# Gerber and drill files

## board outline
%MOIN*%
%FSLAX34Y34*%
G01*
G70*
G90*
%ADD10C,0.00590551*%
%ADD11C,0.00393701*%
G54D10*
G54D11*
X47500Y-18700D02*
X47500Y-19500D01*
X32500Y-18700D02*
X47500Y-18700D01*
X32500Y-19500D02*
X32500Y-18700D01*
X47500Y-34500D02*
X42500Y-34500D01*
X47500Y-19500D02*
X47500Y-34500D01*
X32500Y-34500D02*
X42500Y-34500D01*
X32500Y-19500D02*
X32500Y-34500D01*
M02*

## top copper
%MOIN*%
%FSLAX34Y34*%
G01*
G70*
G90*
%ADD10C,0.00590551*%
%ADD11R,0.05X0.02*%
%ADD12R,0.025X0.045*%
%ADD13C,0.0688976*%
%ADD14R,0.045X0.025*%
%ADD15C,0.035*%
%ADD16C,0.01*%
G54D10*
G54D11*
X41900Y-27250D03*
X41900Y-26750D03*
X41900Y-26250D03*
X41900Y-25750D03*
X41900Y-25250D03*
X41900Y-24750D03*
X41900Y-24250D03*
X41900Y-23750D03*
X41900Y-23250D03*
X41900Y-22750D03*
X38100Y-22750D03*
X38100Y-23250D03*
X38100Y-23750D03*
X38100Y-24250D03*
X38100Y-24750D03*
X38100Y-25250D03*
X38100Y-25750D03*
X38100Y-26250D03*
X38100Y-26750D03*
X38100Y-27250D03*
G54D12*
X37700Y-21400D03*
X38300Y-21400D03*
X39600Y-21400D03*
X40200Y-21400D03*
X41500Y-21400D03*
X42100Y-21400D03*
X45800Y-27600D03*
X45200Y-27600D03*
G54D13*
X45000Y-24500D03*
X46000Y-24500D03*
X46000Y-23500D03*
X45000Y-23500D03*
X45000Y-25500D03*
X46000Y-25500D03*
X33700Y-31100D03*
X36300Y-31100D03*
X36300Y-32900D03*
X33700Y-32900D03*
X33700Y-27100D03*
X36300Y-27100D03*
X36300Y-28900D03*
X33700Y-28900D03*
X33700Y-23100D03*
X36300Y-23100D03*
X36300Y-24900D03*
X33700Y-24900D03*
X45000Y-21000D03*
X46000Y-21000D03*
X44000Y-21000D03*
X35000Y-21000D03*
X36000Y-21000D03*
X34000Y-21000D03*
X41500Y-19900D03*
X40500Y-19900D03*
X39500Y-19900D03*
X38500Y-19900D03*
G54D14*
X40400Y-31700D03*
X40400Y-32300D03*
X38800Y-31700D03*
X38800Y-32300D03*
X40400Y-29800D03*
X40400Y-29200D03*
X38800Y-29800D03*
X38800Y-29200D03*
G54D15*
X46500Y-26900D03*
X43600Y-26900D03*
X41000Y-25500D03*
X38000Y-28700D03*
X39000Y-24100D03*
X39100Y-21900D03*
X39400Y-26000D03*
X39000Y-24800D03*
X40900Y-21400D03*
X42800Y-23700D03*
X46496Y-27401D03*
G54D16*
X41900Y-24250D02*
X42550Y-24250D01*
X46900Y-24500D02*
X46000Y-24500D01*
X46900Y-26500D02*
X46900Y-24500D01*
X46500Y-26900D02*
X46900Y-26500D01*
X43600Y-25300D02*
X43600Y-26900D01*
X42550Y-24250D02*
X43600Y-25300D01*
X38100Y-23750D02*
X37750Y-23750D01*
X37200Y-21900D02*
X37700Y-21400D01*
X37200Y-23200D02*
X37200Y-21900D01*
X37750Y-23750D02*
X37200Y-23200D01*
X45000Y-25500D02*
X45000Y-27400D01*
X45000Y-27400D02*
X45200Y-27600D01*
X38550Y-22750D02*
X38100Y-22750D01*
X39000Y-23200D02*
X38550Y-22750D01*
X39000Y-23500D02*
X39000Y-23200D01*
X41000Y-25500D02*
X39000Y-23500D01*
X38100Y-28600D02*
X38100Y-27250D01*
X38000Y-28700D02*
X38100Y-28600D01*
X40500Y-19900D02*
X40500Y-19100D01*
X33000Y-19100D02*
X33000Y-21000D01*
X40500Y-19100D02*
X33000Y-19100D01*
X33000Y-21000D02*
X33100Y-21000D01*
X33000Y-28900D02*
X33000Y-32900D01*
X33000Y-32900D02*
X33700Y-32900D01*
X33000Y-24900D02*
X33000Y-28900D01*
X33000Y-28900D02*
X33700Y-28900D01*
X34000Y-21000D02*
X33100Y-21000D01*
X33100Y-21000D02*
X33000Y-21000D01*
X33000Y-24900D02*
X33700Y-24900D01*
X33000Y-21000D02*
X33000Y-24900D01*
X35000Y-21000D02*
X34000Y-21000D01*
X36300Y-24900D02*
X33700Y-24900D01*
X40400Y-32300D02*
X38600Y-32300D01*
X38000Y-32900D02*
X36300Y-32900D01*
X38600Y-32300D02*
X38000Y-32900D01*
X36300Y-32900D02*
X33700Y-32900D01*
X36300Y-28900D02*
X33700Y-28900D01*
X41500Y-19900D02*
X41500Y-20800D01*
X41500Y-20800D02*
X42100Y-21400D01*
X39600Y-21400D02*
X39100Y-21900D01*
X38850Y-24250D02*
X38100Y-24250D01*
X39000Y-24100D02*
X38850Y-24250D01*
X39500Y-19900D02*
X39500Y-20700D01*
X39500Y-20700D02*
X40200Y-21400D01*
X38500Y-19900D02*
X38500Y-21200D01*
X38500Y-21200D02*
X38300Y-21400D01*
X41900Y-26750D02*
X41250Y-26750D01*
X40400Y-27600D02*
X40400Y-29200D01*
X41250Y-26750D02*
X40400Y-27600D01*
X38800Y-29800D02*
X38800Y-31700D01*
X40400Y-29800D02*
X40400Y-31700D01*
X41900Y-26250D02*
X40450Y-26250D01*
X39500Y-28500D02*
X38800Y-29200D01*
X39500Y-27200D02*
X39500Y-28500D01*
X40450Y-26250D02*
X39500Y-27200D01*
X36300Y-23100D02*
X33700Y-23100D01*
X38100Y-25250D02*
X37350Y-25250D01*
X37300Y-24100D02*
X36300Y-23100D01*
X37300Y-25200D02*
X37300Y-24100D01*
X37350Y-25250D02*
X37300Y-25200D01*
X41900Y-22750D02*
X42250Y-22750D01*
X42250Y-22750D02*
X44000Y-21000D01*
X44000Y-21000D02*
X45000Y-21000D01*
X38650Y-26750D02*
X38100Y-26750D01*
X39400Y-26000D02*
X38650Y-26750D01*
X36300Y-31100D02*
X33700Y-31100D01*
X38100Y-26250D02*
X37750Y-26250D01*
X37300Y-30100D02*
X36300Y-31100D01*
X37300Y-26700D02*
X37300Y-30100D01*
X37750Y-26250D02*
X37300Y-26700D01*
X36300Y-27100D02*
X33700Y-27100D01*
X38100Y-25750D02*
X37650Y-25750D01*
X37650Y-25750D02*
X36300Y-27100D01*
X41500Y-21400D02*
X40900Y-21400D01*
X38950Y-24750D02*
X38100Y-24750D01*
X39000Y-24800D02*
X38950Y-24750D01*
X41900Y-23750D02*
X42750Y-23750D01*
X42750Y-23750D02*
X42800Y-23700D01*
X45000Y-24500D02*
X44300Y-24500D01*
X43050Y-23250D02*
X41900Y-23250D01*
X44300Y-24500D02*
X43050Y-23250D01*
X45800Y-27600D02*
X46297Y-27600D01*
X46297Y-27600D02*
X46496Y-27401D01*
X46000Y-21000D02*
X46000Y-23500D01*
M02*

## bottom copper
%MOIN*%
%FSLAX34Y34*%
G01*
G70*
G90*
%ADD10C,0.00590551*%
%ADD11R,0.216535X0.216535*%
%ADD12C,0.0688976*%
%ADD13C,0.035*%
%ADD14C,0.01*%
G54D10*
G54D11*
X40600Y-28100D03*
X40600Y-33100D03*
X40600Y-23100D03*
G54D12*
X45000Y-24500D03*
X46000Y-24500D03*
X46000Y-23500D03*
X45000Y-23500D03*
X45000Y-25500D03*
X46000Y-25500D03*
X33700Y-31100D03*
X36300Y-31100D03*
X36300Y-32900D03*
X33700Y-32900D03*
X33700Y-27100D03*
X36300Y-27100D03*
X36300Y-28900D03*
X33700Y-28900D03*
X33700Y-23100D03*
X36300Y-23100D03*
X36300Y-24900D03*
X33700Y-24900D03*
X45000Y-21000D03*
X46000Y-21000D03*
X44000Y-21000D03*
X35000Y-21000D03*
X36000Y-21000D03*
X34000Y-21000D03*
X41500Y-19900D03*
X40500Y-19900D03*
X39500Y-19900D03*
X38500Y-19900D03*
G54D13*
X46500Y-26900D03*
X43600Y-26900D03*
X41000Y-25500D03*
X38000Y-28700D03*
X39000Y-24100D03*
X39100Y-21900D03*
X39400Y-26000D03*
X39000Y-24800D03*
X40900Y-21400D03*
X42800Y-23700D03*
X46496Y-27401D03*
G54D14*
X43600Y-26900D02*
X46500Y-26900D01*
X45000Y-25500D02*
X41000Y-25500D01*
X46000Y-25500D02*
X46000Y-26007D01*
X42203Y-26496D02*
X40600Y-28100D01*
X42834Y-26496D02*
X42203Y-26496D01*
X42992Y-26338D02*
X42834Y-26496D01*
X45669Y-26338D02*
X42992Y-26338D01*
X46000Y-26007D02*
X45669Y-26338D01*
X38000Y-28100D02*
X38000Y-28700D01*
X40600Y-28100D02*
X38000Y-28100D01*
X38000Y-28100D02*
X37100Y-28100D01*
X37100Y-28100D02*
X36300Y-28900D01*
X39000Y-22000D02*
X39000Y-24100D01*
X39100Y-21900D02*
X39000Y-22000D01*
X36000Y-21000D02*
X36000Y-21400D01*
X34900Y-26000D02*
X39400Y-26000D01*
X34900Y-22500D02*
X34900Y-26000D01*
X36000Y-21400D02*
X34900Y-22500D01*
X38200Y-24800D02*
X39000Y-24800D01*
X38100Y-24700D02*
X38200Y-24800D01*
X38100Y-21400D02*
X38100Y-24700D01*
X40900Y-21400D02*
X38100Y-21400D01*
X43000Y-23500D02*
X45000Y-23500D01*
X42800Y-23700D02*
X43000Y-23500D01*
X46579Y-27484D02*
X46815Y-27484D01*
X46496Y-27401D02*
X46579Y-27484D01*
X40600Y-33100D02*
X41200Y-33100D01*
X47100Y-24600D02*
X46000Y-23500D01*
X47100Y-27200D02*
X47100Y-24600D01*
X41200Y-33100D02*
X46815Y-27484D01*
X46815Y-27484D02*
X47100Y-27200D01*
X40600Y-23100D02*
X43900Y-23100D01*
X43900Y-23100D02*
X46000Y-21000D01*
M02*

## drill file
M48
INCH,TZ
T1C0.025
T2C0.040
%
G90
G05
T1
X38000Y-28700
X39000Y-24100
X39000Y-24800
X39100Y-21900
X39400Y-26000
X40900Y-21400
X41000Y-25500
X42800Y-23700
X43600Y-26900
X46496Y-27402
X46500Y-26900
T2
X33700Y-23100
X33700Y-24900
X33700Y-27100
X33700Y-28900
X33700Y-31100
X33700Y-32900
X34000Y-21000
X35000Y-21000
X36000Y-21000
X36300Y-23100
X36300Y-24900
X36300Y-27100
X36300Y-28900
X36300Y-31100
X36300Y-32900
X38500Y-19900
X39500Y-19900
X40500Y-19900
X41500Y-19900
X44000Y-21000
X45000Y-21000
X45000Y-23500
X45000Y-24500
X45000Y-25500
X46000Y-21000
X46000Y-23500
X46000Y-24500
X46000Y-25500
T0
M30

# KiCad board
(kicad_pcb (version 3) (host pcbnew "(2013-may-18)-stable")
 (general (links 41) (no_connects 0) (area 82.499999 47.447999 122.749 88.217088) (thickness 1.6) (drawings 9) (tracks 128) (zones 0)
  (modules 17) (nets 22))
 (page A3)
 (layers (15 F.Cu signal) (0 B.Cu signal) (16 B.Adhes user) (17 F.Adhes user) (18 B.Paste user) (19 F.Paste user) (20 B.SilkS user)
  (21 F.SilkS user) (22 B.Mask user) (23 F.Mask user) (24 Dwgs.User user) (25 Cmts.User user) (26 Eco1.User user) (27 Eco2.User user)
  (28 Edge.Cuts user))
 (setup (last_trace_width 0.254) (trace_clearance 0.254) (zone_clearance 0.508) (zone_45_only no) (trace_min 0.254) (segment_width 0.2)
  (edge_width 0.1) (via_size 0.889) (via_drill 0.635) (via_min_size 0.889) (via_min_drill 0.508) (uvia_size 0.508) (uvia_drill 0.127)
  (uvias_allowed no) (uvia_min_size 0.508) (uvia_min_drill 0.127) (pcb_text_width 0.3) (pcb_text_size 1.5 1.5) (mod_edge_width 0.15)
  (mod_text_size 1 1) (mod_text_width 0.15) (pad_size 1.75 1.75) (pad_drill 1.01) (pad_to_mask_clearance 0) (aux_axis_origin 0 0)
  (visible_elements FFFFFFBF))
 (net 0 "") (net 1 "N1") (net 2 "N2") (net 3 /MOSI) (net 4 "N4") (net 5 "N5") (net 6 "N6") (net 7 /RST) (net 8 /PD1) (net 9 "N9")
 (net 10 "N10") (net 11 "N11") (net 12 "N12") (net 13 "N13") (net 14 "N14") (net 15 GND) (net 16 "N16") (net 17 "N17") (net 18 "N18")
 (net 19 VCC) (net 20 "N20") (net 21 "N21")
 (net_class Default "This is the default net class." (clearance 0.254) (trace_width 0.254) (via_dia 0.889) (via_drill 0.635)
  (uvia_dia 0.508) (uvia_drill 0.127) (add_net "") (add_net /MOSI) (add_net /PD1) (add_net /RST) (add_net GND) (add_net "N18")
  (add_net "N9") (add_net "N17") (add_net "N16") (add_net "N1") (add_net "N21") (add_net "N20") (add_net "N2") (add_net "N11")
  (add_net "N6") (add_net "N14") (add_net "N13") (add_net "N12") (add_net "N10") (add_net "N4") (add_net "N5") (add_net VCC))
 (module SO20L (layer F.Cu) (at 101.6 63.5 270)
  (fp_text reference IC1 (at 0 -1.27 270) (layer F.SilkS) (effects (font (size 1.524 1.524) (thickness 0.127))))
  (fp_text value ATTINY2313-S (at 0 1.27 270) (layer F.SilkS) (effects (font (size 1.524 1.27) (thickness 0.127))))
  (pad 11 smd rect (at 5.715 -4.826 270) (size 0.508 1.27) (layers F.Cu F.Paste F.Mask))
  (pad 12 smd rect (at 4.445 -4.826 270) (size 0.508 1.27) (layers F.Cu F.Paste F.Mask) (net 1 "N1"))
  (pad 13 smd rect (at 3.175 -4.826 270) (size 0.508 1.27) (layers F.Cu F.Paste F.Mask) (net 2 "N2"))
  (pad 14 smd rect (at 1.905 -4.826 270) (size 0.508 1.27) (layers F.Cu F.Paste F.Mask))
  (pad 15 smd rect (at 0.635 -4.826 270) (size 0.508 1.27) (layers F.Cu F.Paste F.Mask))
  (pad 16 smd rect (at -0.635 -4.826 270) (size 0.508 1.27) (layers F.Cu F.Paste F.Mask))
  (pad 17 smd rect (at -1.905 -4.826 270) (size 0.508 1.27) (layers F.Cu F.Paste F.Mask) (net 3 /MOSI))
  (pad 18 smd rect (at -3.175 -4.826 270) (size 0.508 1.27) (layers F.Cu F.Paste F.Mask) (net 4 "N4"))
  (pad 19 smd rect (at -4.445 -4.826 270) (size 0.508 1.27) (layers F.Cu F.Paste F.Mask) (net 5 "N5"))
  (pad 20 smd rect (at -5.715 -4.826 270) (size 0.508 1.27) (layers F.Cu F.Paste F.Mask) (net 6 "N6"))
  (pad 1 smd rect (at -5.715 4.826 270) (size 0.508 1.27) (layers F.Cu F.Paste F.Mask) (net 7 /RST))
  (pad 2 smd rect (at -4.445 4.826 270) (size 0.508 1.27) (layers F.Cu F.Paste F.Mask))
  (pad 3 smd rect (at -3.175 4.826 270) (size 0.508 1.27) (layers F.Cu F.Paste F.Mask) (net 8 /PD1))
  (pad 4 smd rect (at -1.905 4.826 270) (size 0.508 1.27) (layers F.Cu F.Paste F.Mask) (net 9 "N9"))
  (pad 5 smd rect (at -0.635 4.826 270) (size 0.508 1.27) (layers F.Cu F.Paste F.Mask) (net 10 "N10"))
  (pad 6 smd rect (at 0.635 4.826 270) (size 0.508 1.27) (layers F.Cu F.Paste F.Mask) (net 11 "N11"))
  (pad 7 smd rect (at 1.905 4.826 270) (size 0.508 1.27) (layers F.Cu F.Paste F.Mask) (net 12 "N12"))
  (pad 8 smd rect (at 3.175 4.826 270) (size 0.508 1.27) (layers F.Cu F.Paste F.Mask) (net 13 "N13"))
  (pad 9 smd rect (at 4.445 4.826 270) (size 0.508 1.27) (layers F.Cu F.Paste F.Mask) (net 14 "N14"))
  (pad 10 smd rect (at 5.715 4.826 270) (size 0.508 1.27) (layers F.Cu F.Paste F.Mask) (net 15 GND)))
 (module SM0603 (layer F.Cu) (at 96.52 54.356)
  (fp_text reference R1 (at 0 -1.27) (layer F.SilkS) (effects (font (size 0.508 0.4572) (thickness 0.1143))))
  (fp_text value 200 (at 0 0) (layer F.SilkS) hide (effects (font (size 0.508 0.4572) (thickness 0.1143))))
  (pad 1 smd rect (at -0.762 0) (size 0.635 1.143) (layers F.Cu F.Paste F.Mask) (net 8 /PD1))
  (pad 2 smd rect (at 0.762 0) (size 0.635 1.143) (layers F.Cu F.Paste F.Mask) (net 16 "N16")))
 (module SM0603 (layer F.Cu) (at 101.346 54.356)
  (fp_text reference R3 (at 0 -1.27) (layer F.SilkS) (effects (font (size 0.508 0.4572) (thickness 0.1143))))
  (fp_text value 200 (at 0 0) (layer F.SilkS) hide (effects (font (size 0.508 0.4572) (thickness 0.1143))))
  (pad 1 smd rect (at -0.762 0) (size 0.635 1.143) (layers F.Cu F.Paste F.Mask) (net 9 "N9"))
  (pad 2 smd rect (at 0.762 0) (size 0.635 1.143) (layers F.Cu F.Paste F.Mask) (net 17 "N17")))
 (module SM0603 (layer F.Cu) (at 106.172 54.356)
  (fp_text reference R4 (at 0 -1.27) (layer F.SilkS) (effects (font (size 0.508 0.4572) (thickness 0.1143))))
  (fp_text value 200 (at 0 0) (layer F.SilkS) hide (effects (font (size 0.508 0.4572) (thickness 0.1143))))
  (pad 1 smd rect (at -0.762 0) (size 0.635 1.143) (layers F.Cu F.Paste F.Mask) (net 10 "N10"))
  (pad 2 smd rect (at 0.762 0) (size 0.635 1.143) (layers F.Cu F.Paste F.Mask) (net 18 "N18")))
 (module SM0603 (layer F.Cu) (at 115.57 70.104 180)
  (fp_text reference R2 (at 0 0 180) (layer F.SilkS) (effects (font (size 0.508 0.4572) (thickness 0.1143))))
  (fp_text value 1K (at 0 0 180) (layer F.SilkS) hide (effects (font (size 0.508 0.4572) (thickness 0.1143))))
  (pad 1 smd rect (at -0.762 0 180) (size 0.635 1.143) (layers F.Cu F.Paste F.Mask) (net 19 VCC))
  (pad 2 smd rect (at 0.762 0 180) (size 0.635 1.143) (layers F.Cu F.Paste F.Mask) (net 7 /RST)))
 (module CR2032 (layer B.Cu) (at 103.124 71.374 90)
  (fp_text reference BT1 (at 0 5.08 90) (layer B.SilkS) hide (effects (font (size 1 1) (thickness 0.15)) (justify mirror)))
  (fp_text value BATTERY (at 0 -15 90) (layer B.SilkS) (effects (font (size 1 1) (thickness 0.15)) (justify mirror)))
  (pad 2 smd rect (at 0 0 90) (size 5.5 5.5) (layers B.Cu B.Paste B.Mask) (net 15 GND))
  (pad 1 smd rect (at -12.7 0 90) (size 5.5 5.5) (layers B.Cu B.Paste B.Mask) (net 19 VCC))
  (pad 1 smd rect (at 12.7 0 90) (size 5.5 5.5) (layers B.Cu B.Paste B.Mask) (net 19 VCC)))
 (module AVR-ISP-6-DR (layer F.Cu) (at 115.57 62.23 270)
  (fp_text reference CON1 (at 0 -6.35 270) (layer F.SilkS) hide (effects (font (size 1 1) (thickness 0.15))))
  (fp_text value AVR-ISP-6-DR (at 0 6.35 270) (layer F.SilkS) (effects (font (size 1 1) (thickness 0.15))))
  (pad 3 thru_hole circle (at 0 1.27 270) (size 1.75 1.75) (drill 1.01) (layers *.Cu *.Mask F.SilkS) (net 5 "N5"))
  (pad 4 thru_hole circle (at 0 -1.27 270) (size 1.75 1.75) (drill 1.01) (layers *.Cu *.Mask F.SilkS) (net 3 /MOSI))
  (pad 2 thru_hole circle (at -2.54 -1.27 270) (size 1.75 1.75) (drill 1.01) (layers *.Cu *.Mask F.SilkS) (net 19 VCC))
  (pad 1 thru_hole circle (at -2.54 1.27 270) (size 1.75 1.75) (drill 1.01) (layers *.Cu *.Mask F.SilkS) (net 4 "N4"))
  (pad 5 thru_hole circle (at 2.54 1.27 270) (size 1.75 1.75) (drill 1.01) (layers *.Cu *.Mask F.SilkS) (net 7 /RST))
  (pad 6 thru_hole circle (at 2.54 -1.27 270) (size 1.75 1.75) (drill 1.01) (layers *.Cu *.Mask F.SilkS) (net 15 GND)))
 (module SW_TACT (layer F.Cu) (at 88.9 81.28)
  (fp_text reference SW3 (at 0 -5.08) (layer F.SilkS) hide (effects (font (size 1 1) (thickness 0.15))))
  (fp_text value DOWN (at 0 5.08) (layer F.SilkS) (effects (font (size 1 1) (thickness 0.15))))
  (pad 1 thru_hole circle (at -3.302 -2.286) (size 1.75 1.75) (drill 1.01) (layers *.Cu *.Mask F.SilkS) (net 13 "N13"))
  (pad 1 thru_hole circle (at 3.302 -2.286) (size 1.75 1.75) (drill 1.01) (layers *.Cu *.Mask F.SilkS) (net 13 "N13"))
  (pad 2 thru_hole circle (at 3.302 2.286) (size 1.75 1.75) (drill 1.01) (layers *.Cu *.Mask F.SilkS) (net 15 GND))
  (pad 2 thru_hole circle (at -3.302 2.286) (size 1.75 1.75) (drill 1.01) (layers *.Cu *.Mask F.SilkS) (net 15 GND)))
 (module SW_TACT (layer F.Cu) (at 88.9 71.12)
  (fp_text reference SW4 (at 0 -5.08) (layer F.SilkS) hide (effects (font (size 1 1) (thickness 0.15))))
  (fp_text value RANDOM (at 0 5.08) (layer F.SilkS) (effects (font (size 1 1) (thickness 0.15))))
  (pad 1 thru_hole circle (at -3.302 -2.286) (size 1.75 1.75) (drill 1.01) (layers *.Cu *.Mask F.SilkS) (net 12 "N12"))
  (pad 1 thru_hole circle (at 3.302 -2.286) (size 1.75 1.75) (drill 1.01) (layers *.Cu *.Mask F.SilkS) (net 12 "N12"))
  (pad 2 thru_hole circle (at 3.302 2.286) (size 1.75 1.75) (drill 1.01) (layers *.Cu *.Mask F.SilkS) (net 15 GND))
  (pad 2 thru_hole circle (at -3.302 2.286) (size 1.75 1.75) (drill 1.01) (layers *.Cu *.Mask F.SilkS) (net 15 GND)))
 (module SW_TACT (layer F.Cu) (at 88.9 60.96)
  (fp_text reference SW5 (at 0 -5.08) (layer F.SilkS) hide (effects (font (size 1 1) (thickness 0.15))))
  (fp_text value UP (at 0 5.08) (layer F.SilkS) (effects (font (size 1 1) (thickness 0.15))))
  (pad 1 thru_hole circle (at -3.302 -2.286) (size 1.75 1.75) (drill 1.01) (layers *.Cu *.Mask F.SilkS) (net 11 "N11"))
  (pad 1 thru_hole circle (at 3.302 -2.286) (size 1.75 1.75) (drill 1.01) (layers *.Cu *.Mask F.SilkS) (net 11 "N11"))
  (pad 2 thru_hole circle (at 3.302 2.286) (size 1.75 1.75) (drill 1.01) (layers *.Cu *.Mask F.SilkS) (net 15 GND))
  (pad 2 thru_hole circle (at -3.302 2.286) (size 1.75 1.75) (drill 1.01) (layers *.Cu *.Mask F.SilkS) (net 15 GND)))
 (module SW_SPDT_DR (layer F.Cu) (at 114.3 53.34 180)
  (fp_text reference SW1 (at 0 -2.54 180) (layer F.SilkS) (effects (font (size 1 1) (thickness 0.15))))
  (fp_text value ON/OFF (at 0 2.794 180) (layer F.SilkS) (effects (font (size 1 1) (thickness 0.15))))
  (pad 2 thru_hole circle (at 0 0 180) (size 1.75 1.75) (drill 1.01) (layers *.Cu *.Mask F.SilkS) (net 6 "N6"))
  (pad 1 thru_hole circle (at -2.54 0 180) (size 1.75 1.75) (drill 1.01) (layers *.Cu *.Mask F.SilkS) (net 19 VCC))
  (pad 2 thru_hole circle (at 2.54 0 180) (size 1.75 1.75) (drill 1.01) (layers *.Cu *.Mask F.SilkS) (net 6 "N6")))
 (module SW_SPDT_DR (layer F.Cu) (at 88.9 53.34 180)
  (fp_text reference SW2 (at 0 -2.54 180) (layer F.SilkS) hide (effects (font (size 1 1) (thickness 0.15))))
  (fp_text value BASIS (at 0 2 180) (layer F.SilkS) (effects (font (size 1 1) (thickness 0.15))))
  (pad 2 thru_hole circle (at 0 0 180) (size 1.75 1.75) (drill 1.01) (layers *.Cu *.Mask F.SilkS) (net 15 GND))
  (pad 1 thru_hole circle (at -2.54 0 180) (size 1.75 1.75) (drill 1.01) (layers *.Cu *.Mask F.SilkS) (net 14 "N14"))
  (pad 2 thru_hole circle (at 2.54 0 180) (size 1.75 1.75) (drill 1.01) (layers *.Cu *.Mask F.SilkS) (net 15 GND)))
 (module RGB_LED (layer F.Cu) (at 101.6 50.546 180)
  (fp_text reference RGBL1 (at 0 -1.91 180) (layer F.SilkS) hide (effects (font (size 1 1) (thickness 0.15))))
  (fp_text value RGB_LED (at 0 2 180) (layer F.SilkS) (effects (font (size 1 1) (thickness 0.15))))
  (pad 1 thru_hole circle (at -3.81 0 180) (size 1.75 1.75) (drill 1.01) (layers *.Cu *.Mask F.SilkS) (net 18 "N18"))
  (pad 2 thru_hole circle (at -1.27 0 180) (size 1.75 1.75) (drill 1.01) (layers *.Cu *.Mask F.SilkS) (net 15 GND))
  (pad 3 thru_hole circle (at 1.27 0 180) (size 1.75 1.75) (drill 1.01) (layers *.Cu *.Mask F.SilkS) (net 17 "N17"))
  (pad 4 thru_hole circle (at 3.81 0 180) (size 1.75 1.75) (drill 1.01) (layers *.Cu *.Mask F.SilkS) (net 16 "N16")))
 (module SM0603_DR (layer F.Cu) (at 102.616 81.28 270)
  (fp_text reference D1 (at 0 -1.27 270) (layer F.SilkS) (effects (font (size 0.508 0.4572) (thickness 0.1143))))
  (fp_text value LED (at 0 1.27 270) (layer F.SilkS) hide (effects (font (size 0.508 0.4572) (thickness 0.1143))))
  (pad 1 smd rect (at -0.762 0 270) (size 0.635 1.143) (layers F.Cu F.Paste F.Mask) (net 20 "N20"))
  (pad 2 smd rect (at 0.762 0 270) (size 0.635 1.143) (layers F.Cu F.Paste F.Mask) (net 15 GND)))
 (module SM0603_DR (layer F.Cu) (at 98.552 81.28 270)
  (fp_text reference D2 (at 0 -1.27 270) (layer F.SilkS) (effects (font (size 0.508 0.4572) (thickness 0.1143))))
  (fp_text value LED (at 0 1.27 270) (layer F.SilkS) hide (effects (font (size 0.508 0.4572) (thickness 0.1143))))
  (pad 1 smd rect (at -0.762 0 270) (size 0.635 1.143) (layers F.Cu F.Paste F.Mask) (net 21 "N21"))
  (pad 2 smd rect (at 0.762 0 270) (size 0.635 1.143) (layers F.Cu F.Paste F.Mask) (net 15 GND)))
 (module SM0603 (layer F.Cu) (at 102.616 74.93 90)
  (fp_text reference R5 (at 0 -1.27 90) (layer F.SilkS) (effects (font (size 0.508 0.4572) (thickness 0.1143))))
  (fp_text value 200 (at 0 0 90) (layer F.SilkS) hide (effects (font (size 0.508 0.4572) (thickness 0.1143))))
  (pad 1 smd rect (at -0.762 0 90) (size 0.635 1.143) (layers F.Cu F.Paste F.Mask) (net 20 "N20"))
  (pad 2 smd rect (at 0.762 0 90) (size 0.635 1.143) (layers F.Cu F.Paste F.Mask) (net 1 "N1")))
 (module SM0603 (layer F.Cu) (at 98.552 74.93 90)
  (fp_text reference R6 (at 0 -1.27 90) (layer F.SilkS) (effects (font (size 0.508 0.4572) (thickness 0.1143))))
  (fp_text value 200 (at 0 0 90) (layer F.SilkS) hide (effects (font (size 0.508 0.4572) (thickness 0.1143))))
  (pad 1 smd rect (at -0.762 0 90) (size 0.635 1.143) (layers F.Cu F.Paste F.Mask) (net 21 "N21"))
  (pad 2 smd rect (at 0.762 0 90) (size 0.635 1.143) (layers F.Cu F.Paste F.Mask) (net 2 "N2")))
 (gr_line (start 120.65 47.498) (end 120.65 49.53) (angle 90) (layer Edge.Cuts) (width 0.1))
 (gr_line (start 82.55 47.498) (end 120.65 47.498) (angle 90) (layer Edge.Cuts) (width 0.1))
 (gr_line (start 82.55 49.53) (end 82.55 47.498) (angle 90) (layer Edge.Cuts) (width 0.1))
 (gr_line (start 120.65 87.63) (end 107.95 87.63) (angle 90) (layer Edge.Cuts) (width 0.1))
 (gr_line (start 120.65 49.53) (end 120.65 87.63) (angle 90) (layer Edge.Cuts) (width 0.1))
 (gr_line (start 82.55 87.63) (end 107.95 87.63) (angle 90) (layer Edge.Cuts) (width 0.1))
 (gr_line (start 82.55 49.53) (end 82.55 87.63) (angle 90) (layer Edge.Cuts) (width 0.1))
 (segment (start 106.426 61.595) (end 108.077 61.595) (width 0.254) (layer F.Cu) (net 3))
 (segment (start 119.126 62.23) (end 116.84 62.23) (width 0.254) (layer F.Cu) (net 3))
 (segment (start 119.126 67.31) (end 119.126 62.23) (width 0.254) (layer F.Cu) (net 3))
 (segment (start 118.11 68.326) (end 119.126 67.31) (width 0.254) (layer F.Cu) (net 3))
 (via (at 118.11 68.326) (size 0.889) (layers F.Cu B.Cu) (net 3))
 (segment (start 110.744 68.326) (end 118.11 68.326) (width 0.254) (layer B.Cu) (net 3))
 (via (at 110.744 68.326) (size 0.889) (layers F.Cu B.Cu) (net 3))
 (segment (start 110.744 64.262) (end 110.744 68.326) (width 0.254) (layer F.Cu) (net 3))
 (segment (start 108.077 61.595) (end 110.744 64.262) (width 0.254) (layer F.Cu) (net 3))
 (segment (start 96.774 60.325) (end 95.885 60.325) (width 0.254) (layer F.Cu) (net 8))
 (segment (start 94.488 55.626) (end 95.758 54.356) (width 0.254) (layer F.Cu) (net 8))
 (segment (start 94.488 58.928) (end 94.488 55.626) (width 0.254) (layer F.Cu) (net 8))
 (segment (start 95.885 60.325) (end 94.488 58.928) (width 0.254) (layer F.Cu) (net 8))
 (segment (start 114.3 64.77) (end 114.3 69.596) (width 0.254) (layer F.Cu) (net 7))
 (segment (start 114.3 69.596) (end 114.808 70.104) (width 0.254) (layer F.Cu) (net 7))
 (segment (start 114.3 64.77) (end 104.14 64.77) (width 0.254) (layer B.Cu) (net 7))
 (segment (start 97.917 57.785) (end 96.774 57.785) (width 0.254) (layer F.Cu) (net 7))
 (segment (start 99.06 58.928) (end 97.917 57.785) (width 0.254) (layer F.Cu) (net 7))
 (segment (start 99.06 59.69) (end 99.06 58.928) (width 0.254) (layer F.Cu) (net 7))
 (segment (start 104.14 64.77) (end 99.06 59.69) (width 0.254) (layer F.Cu) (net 7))
 (via (at 104.14 64.77) (size 0.889) (layers F.Cu B.Cu) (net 7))
 (segment (start 116.84 64.77) (end 116.84 66.06) (width 0.254) (layer B.Cu) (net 15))
 (segment (start 107.198 67.3) (end 103.124 71.374) (width 0.254) (layer B.Cu) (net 15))
 (segment (start 108.8 67.3) (end 107.198 67.3) (width 0.254) (layer B.Cu) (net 15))
 (segment (start 109.2 66.9) (end 108.8 67.3) (width 0.254) (layer B.Cu) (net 15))
 (segment (start 116 66.9) (end 109.2 66.9) (width 0.254) (layer B.Cu) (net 15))
 (segment (start 116.84 66.06) (end 116 66.9) (width 0.254) (layer B.Cu) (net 15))
 (segment (start 96.52 71.374) (end 96.52 72.898) (width 0.254) (layer B.Cu) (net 15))
 (segment (start 96.774 72.644) (end 96.774 69.215) (width 0.254) (layer F.Cu) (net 15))
 (segment (start 96.52 72.898) (end 96.774 72.644) (width 0.254) (layer F.Cu) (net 15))
 (via (at 96.52 72.898) (size 0.889) (layers F.Cu B.Cu) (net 15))
 (segment (start 103.124 71.374) (end 96.52 71.374) (width 0.254) (layer B.Cu) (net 15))
 (segment (start 96.52 71.374) (end 94.234 71.374) (width 0.254) (layer B.Cu) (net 15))
 (segment (start 94.234 71.374) (end 92.202 73.406) (width 0.254) (layer B.Cu) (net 15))
 (segment (start 102.87 50.546) (end 102.87 48.514) (width 0.254) (layer F.Cu) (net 15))
 (segment (start 83.82 48.514) (end 83.82 53.34) (width 0.254) (layer F.Cu) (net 15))
 (segment (start 102.87 48.514) (end 83.82 48.514) (width 0.254) (layer F.Cu) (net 15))
 (segment (start 83.82 53.34) (end 84.074 53.34) (width 0.254) (layer F.Cu) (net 15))
 (segment (start 83.82 73.406) (end 83.82 83.566) (width 0.254) (layer F.Cu) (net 15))
 (segment (start 83.82 83.566) (end 85.598 83.566) (width 0.254) (layer F.Cu) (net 15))
 (segment (start 83.82 63.246) (end 83.82 73.406) (width 0.254) (layer F.Cu) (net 15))
 (segment (start 83.82 73.406) (end 85.598 73.406) (width 0.254) (layer F.Cu) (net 15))
 (segment (start 86.36 53.34) (end 84.074 53.34) (width 0.254) (layer F.Cu) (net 15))
 (segment (start 84.074 53.34) (end 83.82 53.34) (width 0.254) (layer F.Cu) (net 15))
 (segment (start 83.82 63.246) (end 85.598 63.246) (width 0.254) (layer F.Cu) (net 15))
 (segment (start 83.82 53.34) (end 83.82 63.246) (width 0.254) (layer F.Cu) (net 15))
 (segment (start 88.9 53.34) (end 86.36 53.34) (width 0.254) (layer F.Cu) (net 15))
 (segment (start 92.202 63.246) (end 85.598 63.246) (width 0.254) (layer F.Cu) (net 15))
 (segment (start 102.616 82.042) (end 98.044 82.042) (width 0.254) (layer F.Cu) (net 15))
 (segment (start 96.52 83.566) (end 92.202 83.566) (width 0.254) (layer F.Cu) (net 15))
 (segment (start 98.044 82.042) (end 96.52 83.566) (width 0.254) (layer F.Cu) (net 15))
 (segment (start 92.202 83.566) (end 85.598 83.566) (width 0.254) (layer F.Cu) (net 15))
 (segment (start 92.202 73.406) (end 85.598 73.406) (width 0.254) (layer F.Cu) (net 15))
 (segment (start 105.41 50.546) (end 105.41 52.832) (width 0.254) (layer F.Cu) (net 18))
 (segment (start 105.41 52.832) (end 106.934 54.356) (width 0.254) (layer F.Cu) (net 18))
 (segment (start 100.584 54.356) (end 99.314 55.626) (width 0.254) (layer F.Cu) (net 9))
 (segment (start 98.679 61.595) (end 96.774 61.595) (width 0.254) (layer F.Cu) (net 9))
 (segment (start 99.06 61.214) (end 98.679 61.595) (width 0.254) (layer F.Cu) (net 9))
 (via (at 99.06 61.214) (size 0.889) (layers F.Cu B.Cu) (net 9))
 (segment (start 99.06 55.88) (end 99.06 61.214) (width 0.254) (layer B.Cu) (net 9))
 (segment (start 99.314 55.626) (end 99.06 55.88) (width 0.254) (layer B.Cu) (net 9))
 (via (at 99.314 55.626) (size 0.889) (layers F.Cu B.Cu) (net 9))
 (segment (start 100.33 50.546) (end 100.33 52.578) (width 0.254) (layer F.Cu) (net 17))
 (segment (start 100.33 52.578) (end 102.108 54.356) (width 0.254) (layer F.Cu) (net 17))
 (segment (start 97.79 50.546) (end 97.79 53.848) (width 0.254) (layer F.Cu) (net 16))
 (segment (start 97.79 53.848) (end 97.282 54.356) (width 0.254) (layer F.Cu) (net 16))
 (segment (start 106.426 67.945) (end 104.775 67.945) (width 0.254) (layer F.Cu) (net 1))
 (segment (start 102.616 70.104) (end 102.616 74.168) (width 0.254) (layer F.Cu) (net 1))
 (segment (start 104.775 67.945) (end 102.616 70.104) (width 0.254) (layer F.Cu) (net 1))
 (segment (start 98.552 75.692) (end 98.552 80.518) (width 0.254) (layer F.Cu) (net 21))
 (segment (start 102.616 75.692) (end 102.616 80.518) (width 0.254) (layer F.Cu) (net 20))
 (segment (start 106.426 66.675) (end 102.743 66.675) (width 0.254) (layer F.Cu) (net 2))
 (segment (start 100.33 72.39) (end 98.552 74.168) (width 0.254) (layer F.Cu) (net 2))
 (segment (start 100.33 69.088) (end 100.33 72.39) (width 0.254) (layer F.Cu) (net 2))
 (segment (start 102.743 66.675) (end 100.33 69.088) (width 0.254) (layer F.Cu) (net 2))
 (segment (start 92.202 58.674) (end 85.598 58.674) (width 0.254) (layer F.Cu) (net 11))
 (segment (start 96.774 64.135) (end 94.869 64.135) (width 0.254) (layer F.Cu) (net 11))
 (segment (start 94.742 61.214) (end 92.202 58.674) (width 0.254) (layer F.Cu) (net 11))
 (segment (start 94.742 64.008) (end 94.742 61.214) (width 0.254) (layer F.Cu) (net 11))
 (segment (start 94.869 64.135) (end 94.742 64.008) (width 0.254) (layer F.Cu) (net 11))
 (segment (start 106.426 57.785) (end 107.315 57.785) (width 0.254) (layer F.Cu) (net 6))
 (segment (start 107.315 57.785) (end 111.76 53.34) (width 0.254) (layer F.Cu) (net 6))
 (segment (start 111.76 53.34) (end 114.3 53.34) (width 0.254) (layer F.Cu) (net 6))
 (segment (start 91.44 53.34) (end 91.44 54.356) (width 0.254) (layer B.Cu) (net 14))
 (segment (start 98.171 67.945) (end 96.774 67.945) (width 0.254) (layer F.Cu) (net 14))
 (segment (start 100.076 66.04) (end 98.171 67.945) (width 0.254) (layer F.Cu) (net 14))
 (via (at 100.076 66.04) (size 0.889) (layers F.Cu B.Cu) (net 14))
 (segment (start 88.646 66.04) (end 100.076 66.04) (width 0.254) (layer B.Cu) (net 14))
 (segment (start 88.646 57.15) (end 88.646 66.04) (width 0.254) (layer B.Cu) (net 14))
 (segment (start 91.44 54.356) (end 88.646 57.15) (width 0.254) (layer B.Cu) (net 14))
 (segment (start 92.202 78.994) (end 85.598 78.994) (width 0.254) (layer F.Cu) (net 13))
 (segment (start 96.774 66.675) (end 95.885 66.675) (width 0.254) (layer F.Cu) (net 13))
 (segment (start 94.742 76.454) (end 92.202 78.994) (width 0.254) (layer F.Cu) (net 13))
 (segment (start 94.742 67.818) (end 94.742 76.454) (width 0.254) (layer F.Cu) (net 13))
 (segment (start 95.885 66.675) (end 94.742 67.818) (width 0.254) (layer F.Cu) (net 13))
 (segment (start 92.202 68.834) (end 85.598 68.834) (width 0.254) (layer F.Cu) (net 12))
 (segment (start 96.774 65.405) (end 95.631 65.405) (width 0.254) (layer F.Cu) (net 12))
 (segment (start 95.631 65.405) (end 92.202 68.834) (width 0.254) (layer F.Cu) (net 12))
 (segment (start 105.41 54.356) (end 103.886 54.356) (width 0.254) (layer F.Cu) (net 10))
 (segment (start 98.933 62.865) (end 96.774 62.865) (width 0.254) (layer F.Cu) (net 10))
 (segment (start 99.06 62.992) (end 98.933 62.865) (width 0.254) (layer F.Cu) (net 10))
 (via (at 99.06 62.992) (size 0.889) (layers F.Cu B.Cu) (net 10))
 (segment (start 97.028 62.992) (end 99.06 62.992) (width 0.254) (layer B.Cu) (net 10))
 (segment (start 96.774 62.738) (end 97.028 62.992) (width 0.254) (layer B.Cu) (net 10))
 (segment (start 96.774 54.356) (end 96.774 62.738) (width 0.254) (layer B.Cu) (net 10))
 (segment (start 103.886 54.356) (end 96.774 54.356) (width 0.254) (layer B.Cu) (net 10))
 (via (at 103.886 54.356) (size 0.889) (layers F.Cu B.Cu) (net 10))
 (segment (start 106.426 60.325) (end 108.585 60.325) (width 0.254) (layer F.Cu) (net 4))
 (segment (start 109.22 59.69) (end 114.3 59.69) (width 0.254) (layer B.Cu) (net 4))
 (segment (start 108.712 60.198) (end 109.22 59.69) (width 0.254) (layer B.Cu) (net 4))
 (via (at 108.712 60.198) (size 0.889) (layers F.Cu B.Cu) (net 4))
 (segment (start 108.585 60.325) (end 108.712 60.198) (width 0.254) (layer F.Cu) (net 4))
 (segment (start 114.3 62.23) (end 112.522 62.23) (width 0.254) (layer F.Cu) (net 5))
 (segment (start 109.347 59.055) (end 106.426 59.055) (width 0.254) (layer F.Cu) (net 5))
 (segment (start 112.522 62.23) (end 109.347 59.055) (width 0.254) (layer F.Cu) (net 5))
 (segment (start 116.332 70.104) (end 117.596 70.104) (width 0.254) (layer F.Cu) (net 19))
 (segment (start 118.311 69.811) (end 118.911 69.811) (width 0.254) (layer B.Cu) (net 19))
 (segment (start 118.1 69.6) (end 118.311 69.811) (width 0.254) (layer B.Cu) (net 19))
 (via (at 118.1 69.6) (size 0.889) (layers F.Cu B.Cu) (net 19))
 (segment (start 117.596 70.104) (end 118.1 69.6) (width 0.254) (layer F.Cu) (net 19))
 (segment (start 103.124 84.074) (end 104.648 84.074) (width 0.254) (layer B.Cu) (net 19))
 (segment (start 119.634 62.484) (end 116.84 59.69) (width 0.254) (layer B.Cu) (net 19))
 (segment (start 119.634 69.088) (end 119.634 62.484) (width 0.254) (layer B.Cu) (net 19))
 (segment (start 104.648 84.074) (end 118.911 69.811) (width 0.254) (layer B.Cu) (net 19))
 (segment (start 118.911 69.811) (end 119.634 69.088) (width 0.254) (layer B.Cu) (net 19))
 (segment (start 103.124 58.674) (end 111.506 58.674) (width 0.254) (layer B.Cu) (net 19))
 (segment (start 111.506 58.674) (end 116.84 53.34) (width 0.254) (layer B.Cu) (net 19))
 (segment (start 116.84 53.34) (end 116.84 59.69) (width 0.254) (layer F.Cu) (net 19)))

